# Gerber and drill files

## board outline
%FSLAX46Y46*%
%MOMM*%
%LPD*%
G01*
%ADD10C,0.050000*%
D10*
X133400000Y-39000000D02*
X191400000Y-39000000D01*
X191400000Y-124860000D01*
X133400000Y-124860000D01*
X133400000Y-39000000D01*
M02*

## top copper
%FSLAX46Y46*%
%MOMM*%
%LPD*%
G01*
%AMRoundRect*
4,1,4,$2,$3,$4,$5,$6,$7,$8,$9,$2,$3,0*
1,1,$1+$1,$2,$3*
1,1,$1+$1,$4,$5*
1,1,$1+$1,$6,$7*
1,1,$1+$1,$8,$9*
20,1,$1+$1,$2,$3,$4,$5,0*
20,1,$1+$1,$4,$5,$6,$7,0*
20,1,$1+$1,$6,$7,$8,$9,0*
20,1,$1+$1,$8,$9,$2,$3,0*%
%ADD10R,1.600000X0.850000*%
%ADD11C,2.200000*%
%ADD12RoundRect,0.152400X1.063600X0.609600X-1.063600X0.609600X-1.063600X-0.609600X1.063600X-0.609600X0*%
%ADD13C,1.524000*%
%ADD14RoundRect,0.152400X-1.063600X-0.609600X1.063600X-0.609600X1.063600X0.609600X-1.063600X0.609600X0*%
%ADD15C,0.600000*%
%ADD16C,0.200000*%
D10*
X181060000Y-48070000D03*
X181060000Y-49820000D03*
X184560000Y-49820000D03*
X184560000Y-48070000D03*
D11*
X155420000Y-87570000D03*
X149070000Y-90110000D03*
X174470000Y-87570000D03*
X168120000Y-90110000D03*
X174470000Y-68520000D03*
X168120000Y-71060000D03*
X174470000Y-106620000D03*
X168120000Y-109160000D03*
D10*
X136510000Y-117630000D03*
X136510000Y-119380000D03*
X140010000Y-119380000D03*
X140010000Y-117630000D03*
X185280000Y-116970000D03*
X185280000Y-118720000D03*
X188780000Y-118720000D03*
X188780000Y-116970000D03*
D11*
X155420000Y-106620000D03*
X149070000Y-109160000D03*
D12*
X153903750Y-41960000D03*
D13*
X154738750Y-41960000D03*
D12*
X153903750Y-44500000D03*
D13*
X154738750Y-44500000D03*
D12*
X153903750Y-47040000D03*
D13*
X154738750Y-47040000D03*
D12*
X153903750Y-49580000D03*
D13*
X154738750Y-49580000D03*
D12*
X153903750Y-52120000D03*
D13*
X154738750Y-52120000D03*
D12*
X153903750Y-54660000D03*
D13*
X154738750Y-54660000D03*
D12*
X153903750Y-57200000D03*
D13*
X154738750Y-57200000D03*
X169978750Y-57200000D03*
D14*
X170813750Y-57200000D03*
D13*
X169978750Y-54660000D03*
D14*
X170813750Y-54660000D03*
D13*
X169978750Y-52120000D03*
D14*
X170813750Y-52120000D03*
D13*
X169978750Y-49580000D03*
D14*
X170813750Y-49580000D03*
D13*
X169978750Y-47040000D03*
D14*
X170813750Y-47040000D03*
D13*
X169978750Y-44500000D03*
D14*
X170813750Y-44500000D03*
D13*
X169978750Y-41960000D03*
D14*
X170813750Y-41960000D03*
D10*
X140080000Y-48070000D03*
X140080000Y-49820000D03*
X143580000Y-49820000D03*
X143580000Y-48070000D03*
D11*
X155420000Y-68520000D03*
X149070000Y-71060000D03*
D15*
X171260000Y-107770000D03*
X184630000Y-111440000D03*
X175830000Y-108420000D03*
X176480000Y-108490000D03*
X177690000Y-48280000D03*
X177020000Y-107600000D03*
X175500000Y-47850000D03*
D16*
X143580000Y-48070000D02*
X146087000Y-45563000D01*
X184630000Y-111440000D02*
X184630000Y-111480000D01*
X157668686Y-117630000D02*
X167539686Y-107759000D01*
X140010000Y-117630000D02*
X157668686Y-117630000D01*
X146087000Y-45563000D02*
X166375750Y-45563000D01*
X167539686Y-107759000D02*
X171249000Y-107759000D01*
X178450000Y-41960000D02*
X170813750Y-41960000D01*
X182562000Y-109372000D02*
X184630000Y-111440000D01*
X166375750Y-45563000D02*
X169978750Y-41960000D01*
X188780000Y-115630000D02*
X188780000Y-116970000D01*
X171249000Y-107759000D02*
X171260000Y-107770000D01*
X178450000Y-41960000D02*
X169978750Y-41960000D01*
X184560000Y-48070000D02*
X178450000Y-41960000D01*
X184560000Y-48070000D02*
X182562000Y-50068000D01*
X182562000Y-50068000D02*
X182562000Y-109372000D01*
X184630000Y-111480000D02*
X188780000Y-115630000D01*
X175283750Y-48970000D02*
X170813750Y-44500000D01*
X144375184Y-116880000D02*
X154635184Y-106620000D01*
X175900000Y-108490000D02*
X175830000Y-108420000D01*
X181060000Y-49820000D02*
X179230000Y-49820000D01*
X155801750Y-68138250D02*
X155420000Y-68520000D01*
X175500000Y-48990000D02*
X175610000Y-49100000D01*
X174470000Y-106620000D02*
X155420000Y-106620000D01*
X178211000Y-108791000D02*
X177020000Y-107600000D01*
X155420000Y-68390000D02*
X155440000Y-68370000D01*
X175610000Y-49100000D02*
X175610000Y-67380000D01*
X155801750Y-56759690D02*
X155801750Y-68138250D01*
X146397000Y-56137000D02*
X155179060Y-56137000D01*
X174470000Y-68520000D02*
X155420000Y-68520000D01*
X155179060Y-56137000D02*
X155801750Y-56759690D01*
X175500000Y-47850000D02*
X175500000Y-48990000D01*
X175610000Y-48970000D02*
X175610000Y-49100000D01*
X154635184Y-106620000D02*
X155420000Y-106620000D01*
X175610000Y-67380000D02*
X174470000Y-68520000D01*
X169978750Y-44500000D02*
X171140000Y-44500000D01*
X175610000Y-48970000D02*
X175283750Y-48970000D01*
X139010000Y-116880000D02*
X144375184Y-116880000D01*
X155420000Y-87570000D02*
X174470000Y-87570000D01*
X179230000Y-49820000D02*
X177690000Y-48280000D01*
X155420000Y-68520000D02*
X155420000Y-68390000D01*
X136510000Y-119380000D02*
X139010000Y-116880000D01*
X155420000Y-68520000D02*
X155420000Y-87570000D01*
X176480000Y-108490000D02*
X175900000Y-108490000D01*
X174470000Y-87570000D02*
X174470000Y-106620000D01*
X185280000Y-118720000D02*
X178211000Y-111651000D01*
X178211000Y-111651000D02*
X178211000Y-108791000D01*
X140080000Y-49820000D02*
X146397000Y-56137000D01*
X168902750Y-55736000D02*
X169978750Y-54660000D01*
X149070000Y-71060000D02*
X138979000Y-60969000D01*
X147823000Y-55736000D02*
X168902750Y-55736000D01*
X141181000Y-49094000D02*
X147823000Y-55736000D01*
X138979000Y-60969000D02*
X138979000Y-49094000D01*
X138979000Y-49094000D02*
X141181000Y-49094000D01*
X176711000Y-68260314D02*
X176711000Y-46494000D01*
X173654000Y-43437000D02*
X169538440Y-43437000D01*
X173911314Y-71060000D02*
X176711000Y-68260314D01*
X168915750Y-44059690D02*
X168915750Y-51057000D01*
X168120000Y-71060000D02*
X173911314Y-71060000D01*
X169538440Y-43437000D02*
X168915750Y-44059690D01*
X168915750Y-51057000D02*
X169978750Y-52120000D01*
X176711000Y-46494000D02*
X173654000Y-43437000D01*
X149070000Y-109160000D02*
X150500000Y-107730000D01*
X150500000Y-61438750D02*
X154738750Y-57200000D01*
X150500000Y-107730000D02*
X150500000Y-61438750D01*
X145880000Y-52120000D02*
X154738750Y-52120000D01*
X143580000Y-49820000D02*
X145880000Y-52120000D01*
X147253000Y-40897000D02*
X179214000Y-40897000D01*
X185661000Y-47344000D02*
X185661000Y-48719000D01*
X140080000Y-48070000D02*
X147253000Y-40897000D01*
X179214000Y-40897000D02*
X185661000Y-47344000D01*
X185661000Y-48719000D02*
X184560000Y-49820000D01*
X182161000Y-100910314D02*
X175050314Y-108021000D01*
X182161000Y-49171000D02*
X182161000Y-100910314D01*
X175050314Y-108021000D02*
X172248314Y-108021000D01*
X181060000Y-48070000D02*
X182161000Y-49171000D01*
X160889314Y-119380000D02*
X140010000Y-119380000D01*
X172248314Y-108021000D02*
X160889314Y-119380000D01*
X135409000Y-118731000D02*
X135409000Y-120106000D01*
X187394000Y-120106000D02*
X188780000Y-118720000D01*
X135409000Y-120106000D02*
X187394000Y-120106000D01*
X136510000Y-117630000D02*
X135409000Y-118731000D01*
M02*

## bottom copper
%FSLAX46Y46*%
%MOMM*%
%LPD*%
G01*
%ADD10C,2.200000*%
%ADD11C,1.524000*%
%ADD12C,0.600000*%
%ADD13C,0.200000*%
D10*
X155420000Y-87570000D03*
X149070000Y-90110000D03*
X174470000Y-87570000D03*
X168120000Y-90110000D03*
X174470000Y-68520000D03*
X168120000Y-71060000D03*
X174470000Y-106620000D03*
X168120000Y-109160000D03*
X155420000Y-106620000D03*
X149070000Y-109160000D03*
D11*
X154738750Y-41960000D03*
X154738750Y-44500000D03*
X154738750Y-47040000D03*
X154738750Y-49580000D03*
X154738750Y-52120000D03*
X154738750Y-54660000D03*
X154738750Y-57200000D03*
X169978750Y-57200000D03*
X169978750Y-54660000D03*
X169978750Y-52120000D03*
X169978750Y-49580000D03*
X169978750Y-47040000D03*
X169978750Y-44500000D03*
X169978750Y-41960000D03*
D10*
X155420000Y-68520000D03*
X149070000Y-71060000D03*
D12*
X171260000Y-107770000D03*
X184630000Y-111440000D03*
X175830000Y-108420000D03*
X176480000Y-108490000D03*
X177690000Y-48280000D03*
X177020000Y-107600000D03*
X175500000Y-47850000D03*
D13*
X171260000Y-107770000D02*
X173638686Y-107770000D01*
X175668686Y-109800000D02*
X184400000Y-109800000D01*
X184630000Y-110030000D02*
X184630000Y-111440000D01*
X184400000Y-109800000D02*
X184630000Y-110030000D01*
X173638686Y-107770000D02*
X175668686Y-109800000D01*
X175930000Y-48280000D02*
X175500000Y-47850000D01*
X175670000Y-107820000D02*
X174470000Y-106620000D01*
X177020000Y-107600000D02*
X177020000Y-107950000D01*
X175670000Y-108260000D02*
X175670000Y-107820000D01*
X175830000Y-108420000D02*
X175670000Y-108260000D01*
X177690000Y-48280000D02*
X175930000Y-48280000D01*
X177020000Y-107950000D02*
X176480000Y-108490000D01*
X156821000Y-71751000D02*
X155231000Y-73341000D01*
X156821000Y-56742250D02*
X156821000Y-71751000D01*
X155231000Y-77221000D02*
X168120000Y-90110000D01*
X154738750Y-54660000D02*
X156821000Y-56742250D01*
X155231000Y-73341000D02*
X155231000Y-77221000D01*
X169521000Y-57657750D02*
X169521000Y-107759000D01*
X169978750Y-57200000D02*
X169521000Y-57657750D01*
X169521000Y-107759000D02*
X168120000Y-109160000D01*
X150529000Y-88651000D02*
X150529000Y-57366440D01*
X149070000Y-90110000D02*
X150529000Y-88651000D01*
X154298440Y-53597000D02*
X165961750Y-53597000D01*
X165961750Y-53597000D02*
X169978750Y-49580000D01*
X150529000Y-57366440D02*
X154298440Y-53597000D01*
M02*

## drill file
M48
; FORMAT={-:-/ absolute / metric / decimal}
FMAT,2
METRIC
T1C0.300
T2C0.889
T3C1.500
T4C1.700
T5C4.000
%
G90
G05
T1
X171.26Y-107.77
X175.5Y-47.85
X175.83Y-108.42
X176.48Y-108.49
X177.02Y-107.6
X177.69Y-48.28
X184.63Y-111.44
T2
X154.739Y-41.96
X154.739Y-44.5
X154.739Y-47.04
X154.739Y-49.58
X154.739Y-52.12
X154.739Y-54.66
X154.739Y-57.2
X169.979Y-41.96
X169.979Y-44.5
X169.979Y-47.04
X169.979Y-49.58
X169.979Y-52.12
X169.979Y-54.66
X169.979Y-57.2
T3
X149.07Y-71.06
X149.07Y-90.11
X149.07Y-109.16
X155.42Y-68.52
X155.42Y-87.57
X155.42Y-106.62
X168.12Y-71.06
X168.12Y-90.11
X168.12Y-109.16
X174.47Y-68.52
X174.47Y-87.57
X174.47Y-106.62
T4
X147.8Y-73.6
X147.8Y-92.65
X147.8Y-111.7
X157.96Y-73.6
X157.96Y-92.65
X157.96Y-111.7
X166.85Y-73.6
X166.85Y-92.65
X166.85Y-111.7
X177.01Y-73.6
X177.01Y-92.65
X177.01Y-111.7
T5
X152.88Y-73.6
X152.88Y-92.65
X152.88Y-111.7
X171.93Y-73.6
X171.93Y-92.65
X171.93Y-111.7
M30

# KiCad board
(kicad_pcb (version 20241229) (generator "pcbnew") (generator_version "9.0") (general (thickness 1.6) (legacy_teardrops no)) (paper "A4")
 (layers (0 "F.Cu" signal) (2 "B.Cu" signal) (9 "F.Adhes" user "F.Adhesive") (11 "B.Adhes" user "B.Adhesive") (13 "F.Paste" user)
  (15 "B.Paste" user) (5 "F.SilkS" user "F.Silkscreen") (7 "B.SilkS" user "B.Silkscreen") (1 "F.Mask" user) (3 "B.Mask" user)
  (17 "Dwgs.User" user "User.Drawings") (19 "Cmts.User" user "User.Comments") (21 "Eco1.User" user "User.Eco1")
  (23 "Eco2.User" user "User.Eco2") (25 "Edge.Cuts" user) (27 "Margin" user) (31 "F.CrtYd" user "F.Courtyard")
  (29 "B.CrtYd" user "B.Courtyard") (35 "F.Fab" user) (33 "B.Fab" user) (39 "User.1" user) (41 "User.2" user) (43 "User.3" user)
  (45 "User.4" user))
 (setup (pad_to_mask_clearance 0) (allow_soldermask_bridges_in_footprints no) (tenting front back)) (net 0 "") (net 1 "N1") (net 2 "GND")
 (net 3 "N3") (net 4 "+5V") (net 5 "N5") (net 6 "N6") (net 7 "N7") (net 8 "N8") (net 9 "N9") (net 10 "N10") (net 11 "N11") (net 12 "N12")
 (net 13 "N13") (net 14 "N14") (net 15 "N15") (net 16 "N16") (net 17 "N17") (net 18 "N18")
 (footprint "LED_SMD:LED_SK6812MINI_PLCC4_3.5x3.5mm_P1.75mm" (layer "F.Cu") (at 182.81 48.945)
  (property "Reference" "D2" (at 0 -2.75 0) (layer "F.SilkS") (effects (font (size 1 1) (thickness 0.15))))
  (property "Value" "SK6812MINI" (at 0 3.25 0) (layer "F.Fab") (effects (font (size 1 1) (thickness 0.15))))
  (pad "1" smd rect (at -1.75 -0.875) (size 1.6 0.85) (layers "F.Cu" "F.Mask" "F.Paste") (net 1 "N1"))
  (pad "2" smd rect (at -1.75 0.875) (size 1.6 0.85) (layers "F.Cu" "F.Mask" "F.Paste") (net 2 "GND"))
  (pad "3" smd rect (at 1.75 0.875) (size 1.6 0.85) (layers "F.Cu" "F.Mask" "F.Paste") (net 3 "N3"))
  (pad "4" smd rect (at 1.75 -0.875) (size 1.6 0.85) (layers "F.Cu" "F.Mask" "F.Paste") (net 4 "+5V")))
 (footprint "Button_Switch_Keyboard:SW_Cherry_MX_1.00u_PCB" (layer "F.Cu") (at 155.42 87.57)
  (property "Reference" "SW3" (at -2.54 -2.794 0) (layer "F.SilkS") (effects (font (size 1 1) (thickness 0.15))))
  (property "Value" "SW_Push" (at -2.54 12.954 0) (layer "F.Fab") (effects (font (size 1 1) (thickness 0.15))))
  (pad "" np_thru_hole circle (at -7.62 5.08) (size 1.7 1.7) (drill 1.7) (layers "*.Cu" "*.Mask"))
  (pad "" np_thru_hole circle (at -2.54 5.08) (size 4 4) (drill 4) (layers "*.Cu" "*.Mask"))
  (pad "" np_thru_hole circle (at 2.54 5.08) (size 1.7 1.7) (drill 1.7) (layers "*.Cu" "*.Mask"))
  (pad "1" thru_hole circle (at 0 0) (size 2.2 2.2) (drill 1.5) (layers "*.Cu" "*.Mask") (remove_unused_layers no) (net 2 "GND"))
  (pad "2" thru_hole circle (at -6.35 2.54) (size 2.2 2.2) (drill 1.5) (layers "*.Cu" "*.Mask") (remove_unused_layers no) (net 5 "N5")))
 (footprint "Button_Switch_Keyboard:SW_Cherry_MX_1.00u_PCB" (layer "F.Cu") (at 174.47 87.57)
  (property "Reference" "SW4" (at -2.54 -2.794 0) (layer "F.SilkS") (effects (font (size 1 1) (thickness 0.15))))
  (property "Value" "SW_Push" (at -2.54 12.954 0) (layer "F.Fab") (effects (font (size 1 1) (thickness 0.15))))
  (pad "" np_thru_hole circle (at -7.62 5.08) (size 1.7 1.7) (drill 1.7) (layers "*.Cu" "*.Mask"))
  (pad "" np_thru_hole circle (at -2.54 5.08) (size 4 4) (drill 4) (layers "*.Cu" "*.Mask"))
  (pad "" np_thru_hole circle (at 2.54 5.08) (size 1.7 1.7) (drill 1.7) (layers "*.Cu" "*.Mask"))
  (pad "1" thru_hole circle (at 0 0) (size 2.2 2.2) (drill 1.5) (layers "*.Cu" "*.Mask") (remove_unused_layers no) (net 2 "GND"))
  (pad "2" thru_hole circle (at -6.35 2.54) (size 2.2 2.2) (drill 1.5) (layers "*.Cu" "*.Mask") (remove_unused_layers no) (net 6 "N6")))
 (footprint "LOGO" (layer "F.Cu") (at 187.27 93.68 -90)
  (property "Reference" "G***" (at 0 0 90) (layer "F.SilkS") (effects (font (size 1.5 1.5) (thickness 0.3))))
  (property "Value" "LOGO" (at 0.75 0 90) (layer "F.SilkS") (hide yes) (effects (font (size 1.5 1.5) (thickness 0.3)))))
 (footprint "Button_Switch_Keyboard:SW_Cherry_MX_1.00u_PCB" (layer "F.Cu") (at 174.47 68.52)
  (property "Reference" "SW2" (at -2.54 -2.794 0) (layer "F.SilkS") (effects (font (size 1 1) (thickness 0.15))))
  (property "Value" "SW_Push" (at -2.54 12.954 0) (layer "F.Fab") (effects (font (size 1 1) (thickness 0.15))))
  (pad "" np_thru_hole circle (at -7.62 5.08) (size 1.7 1.7) (drill 1.7) (layers "*.Cu" "*.Mask"))
  (pad "" np_thru_hole circle (at -2.54 5.08) (size 4 4) (drill 4) (layers "*.Cu" "*.Mask"))
  (pad "" np_thru_hole circle (at 2.54 5.08) (size 1.7 1.7) (drill 1.7) (layers "*.Cu" "*.Mask"))
  (pad "1" thru_hole circle (at 0 0) (size 2.2 2.2) (drill 1.5) (layers "*.Cu" "*.Mask") (remove_unused_layers no) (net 2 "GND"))
  (pad "2" thru_hole circle (at -6.35 2.54) (size 2.2 2.2) (drill 1.5) (layers "*.Cu" "*.Mask") (remove_unused_layers no) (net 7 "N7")))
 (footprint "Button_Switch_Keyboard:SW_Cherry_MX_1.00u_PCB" (layer "F.Cu") (at 174.47 106.62)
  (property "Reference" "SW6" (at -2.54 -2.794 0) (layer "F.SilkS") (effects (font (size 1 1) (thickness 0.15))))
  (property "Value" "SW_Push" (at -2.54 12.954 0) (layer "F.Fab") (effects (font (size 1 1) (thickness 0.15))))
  (pad "" np_thru_hole circle (at -7.62 5.08) (size 1.7 1.7) (drill 1.7) (layers "*.Cu" "*.Mask"))
  (pad "" np_thru_hole circle (at -2.54 5.08) (size 4 4) (drill 4) (layers "*.Cu" "*.Mask"))
  (pad "" np_thru_hole circle (at 2.54 5.08) (size 1.7 1.7) (drill 1.7) (layers "*.Cu" "*.Mask"))
  (pad "1" thru_hole circle (at 0 0) (size 2.2 2.2) (drill 1.5) (layers "*.Cu" "*.Mask") (remove_unused_layers no) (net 2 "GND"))
  (pad "2" thru_hole circle (at -6.35 2.54) (size 2.2 2.2) (drill 1.5) (layers "*.Cu" "*.Mask") (remove_unused_layers no) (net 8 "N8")))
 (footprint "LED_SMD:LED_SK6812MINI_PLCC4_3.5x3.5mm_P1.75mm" (layer "F.Cu") (at 138.26 118.505)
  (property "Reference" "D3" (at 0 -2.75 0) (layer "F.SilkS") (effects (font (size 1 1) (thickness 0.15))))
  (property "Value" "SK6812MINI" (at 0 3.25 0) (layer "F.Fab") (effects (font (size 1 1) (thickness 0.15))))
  (pad "1" smd rect (at -1.75 -0.875) (size 1.6 0.85) (layers "F.Cu" "F.Mask" "F.Paste") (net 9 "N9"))
  (pad "2" smd rect (at -1.75 0.875) (size 1.6 0.85) (layers "F.Cu" "F.Mask" "F.Paste") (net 2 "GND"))
  (pad "3" smd rect (at 1.75 0.875) (size 1.6 0.85) (layers "F.Cu" "F.Mask" "F.Paste") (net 1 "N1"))
  (pad "4" smd rect (at 1.75 -0.875) (size 1.6 0.85) (layers "F.Cu" "F.Mask" "F.Paste") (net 4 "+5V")))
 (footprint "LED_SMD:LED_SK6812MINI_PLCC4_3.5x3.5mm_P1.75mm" (layer "F.Cu") (at 187.03 117.845)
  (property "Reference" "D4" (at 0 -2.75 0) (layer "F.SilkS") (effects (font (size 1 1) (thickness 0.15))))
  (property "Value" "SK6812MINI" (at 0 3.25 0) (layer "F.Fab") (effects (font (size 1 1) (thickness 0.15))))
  (pad "1" smd rect (at -1.75 -0.875) (size 1.6 0.85) (layers "F.Cu" "F.Mask" "F.Paste") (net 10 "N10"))
  (pad "2" smd rect (at -1.75 0.875) (size 1.6 0.85) (layers "F.Cu" "F.Mask" "F.Paste") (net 2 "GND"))
  (pad "3" smd rect (at 1.75 0.875) (size 1.6 0.85) (layers "F.Cu" "F.Mask" "F.Paste") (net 9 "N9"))
  (pad "4" smd rect (at 1.75 -0.875) (size 1.6 0.85) (layers "F.Cu" "F.Mask" "F.Paste") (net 4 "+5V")))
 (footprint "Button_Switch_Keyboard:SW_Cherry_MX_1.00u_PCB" (layer "F.Cu") (at 155.42 106.62)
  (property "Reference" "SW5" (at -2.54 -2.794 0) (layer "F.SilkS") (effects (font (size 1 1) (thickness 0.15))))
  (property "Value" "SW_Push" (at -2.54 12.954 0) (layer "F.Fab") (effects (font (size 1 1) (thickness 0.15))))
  (pad "" np_thru_hole circle (at -7.62 5.08) (size 1.7 1.7) (drill 1.7) (layers "*.Cu" "*.Mask"))
  (pad "" np_thru_hole circle (at -2.54 5.08) (size 4 4) (drill 4) (layers "*.Cu" "*.Mask"))
  (pad "" np_thru_hole circle (at 2.54 5.08) (size 1.7 1.7) (drill 1.7) (layers "*.Cu" "*.Mask"))
  (pad "1" thru_hole circle (at 0 0) (size 2.2 2.2) (drill 1.5) (layers "*.Cu" "*.Mask") (remove_unused_layers no) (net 2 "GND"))
  (pad "2" thru_hole circle (at -6.35 2.54) (size 2.2 2.2) (drill 1.5) (layers "*.Cu" "*.Mask") (remove_unused_layers no) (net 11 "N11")))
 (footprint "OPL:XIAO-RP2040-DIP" (layer "F.Cu") (at 162.35875 49.58)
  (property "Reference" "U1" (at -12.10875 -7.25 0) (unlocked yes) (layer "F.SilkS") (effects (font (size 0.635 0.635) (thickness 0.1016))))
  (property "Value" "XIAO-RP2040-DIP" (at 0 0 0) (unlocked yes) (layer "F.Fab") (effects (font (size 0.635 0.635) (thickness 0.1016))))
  (pad "1" smd roundrect (at -8.455 -7.62 180) (size 2.432 1.524) (layers "F.Cu" "F.Mask") (roundrect_rratio 0.1) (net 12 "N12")
   (thermal_bridge_angle 45))
  (pad "1" thru_hole circle (at -7.62 -7.62 180) (size 1.524 1.524) (drill 0.889) (layers "*.Cu" "*.Mask") (remove_unused_layers no)
   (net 12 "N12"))
  (pad "2" smd roundrect (at -8.455 -5.08 180) (size 2.432 1.524) (layers "F.Cu" "F.Mask") (roundrect_rratio 0.1) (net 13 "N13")
   (thermal_bridge_angle 45))
  (pad "2" thru_hole circle (at -7.62 -5.08 180) (size 1.524 1.524) (drill 0.889) (layers "*.Cu" "*.Mask") (remove_unused_layers no)
   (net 13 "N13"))
  (pad "3" smd roundrect (at -8.455 -2.54 180) (size 2.432 1.524) (layers "F.Cu" "F.Mask") (roundrect_rratio 0.1) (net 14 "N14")
   (thermal_bridge_angle 45))
  (pad "3" thru_hole circle (at -7.62 -2.54 180) (size 1.524 1.524) (drill 0.889) (layers "*.Cu" "*.Mask") (remove_unused_layers no)
   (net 14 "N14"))
  (pad "4" smd roundrect (at -8.455 0 180) (size 2.432 1.524) (layers "F.Cu" "F.Mask") (roundrect_rratio 0.1) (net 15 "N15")
   (thermal_bridge_angle 45))
  (pad "4" thru_hole circle (at -7.62 0 180) (size 1.524 1.524) (drill 0.889) (layers "*.Cu" "*.Mask") (remove_unused_layers no)
   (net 15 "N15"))
  (pad "5" smd roundrect (at -8.455 2.54 180) (size 2.432 1.524) (layers "F.Cu" "F.Mask") (roundrect_rratio 0.1) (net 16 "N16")
   (thermal_bridge_angle 45))
  (pad "5" thru_hole circle (at -7.62 2.54 180) (size 1.524 1.524) (drill 0.889) (layers "*.Cu" "*.Mask") (remove_unused_layers no)
   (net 16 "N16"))
  (pad "6" smd roundrect (at -8.455 5.08 180) (size 2.432 1.524) (layers "F.Cu" "F.Mask") (roundrect_rratio 0.1) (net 6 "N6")
   (thermal_bridge_angle 45))
  (pad "6" thru_hole circle (at -7.62 5.08 180) (size 1.524 1.524) (drill 0.889) (layers "*.Cu" "*.Mask") (remove_unused_layers no)
   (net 6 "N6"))
  (pad "7" smd roundrect (at -8.455 7.62 180) (size 2.432 1.524) (layers "F.Cu" "F.Mask") (roundrect_rratio 0.1) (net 11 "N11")
   (thermal_bridge_angle 45))
  (pad "7" thru_hole circle (at -7.62 7.62 180) (size 1.524 1.524) (drill 0.889) (layers "*.Cu" "*.Mask") (remove_unused_layers no)
   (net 11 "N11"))
  (pad "8" thru_hole circle (at 7.62 7.62) (size 1.524 1.524) (drill 0.889) (layers "*.Cu" "*.Mask") (remove_unused_layers no) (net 8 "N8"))
  (pad "8" smd roundrect (at 8.455 7.62) (size 2.432 1.524) (layers "F.Cu" "F.Mask") (roundrect_rratio 0.1) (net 8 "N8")
   (thermal_bridge_angle 45))
  (pad "9" thru_hole circle (at 7.62 5.08) (size 1.524 1.524) (drill 0.889) (layers "*.Cu" "*.Mask") (remove_unused_layers no)
   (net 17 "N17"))
  (pad "9" smd roundrect (at 8.455 5.08) (size 2.432 1.524) (layers "F.Cu" "F.Mask") (roundrect_rratio 0.1) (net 17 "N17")
   (thermal_bridge_angle 45))
  (pad "10" thru_hole circle (at 7.62 2.54) (size 1.524 1.524) (drill 0.889) (layers "*.Cu" "*.Mask") (remove_unused_layers no) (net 7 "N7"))
  (pad "10" smd roundrect (at 8.455 2.54) (size 2.432 1.524) (layers "F.Cu" "F.Mask") (roundrect_rratio 0.1) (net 7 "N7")
   (thermal_bridge_angle 45))
  (pad "11" thru_hole circle (at 7.62 0) (size 1.524 1.524) (drill 0.889) (layers "*.Cu" "*.Mask") (remove_unused_layers no) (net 5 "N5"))
  (pad "11" smd roundrect (at 8.455 0) (size 2.432 1.524) (layers "F.Cu" "F.Mask") (roundrect_rratio 0.1) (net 5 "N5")
   (thermal_bridge_angle 45))
  (pad "12" thru_hole circle (at 7.62 -2.54) (size 1.524 1.524) (drill 0.889) (layers "*.Cu" "*.Mask") (remove_unused_layers no)
   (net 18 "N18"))
  (pad "12" smd roundrect (at 8.455 -2.54) (size 2.432 1.524) (layers "F.Cu" "F.Mask") (roundrect_rratio 0.1) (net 18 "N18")
   (thermal_bridge_angle 45))
  (pad "13" thru_hole circle (at 7.62 -5.08) (size 1.524 1.524) (drill 0.889) (layers "*.Cu" "*.Mask") (remove_unused_layers no)
   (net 2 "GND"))
  (pad "13" smd roundrect (at 8.455 -5.08) (size 2.432 1.524) (layers "F.Cu" "F.Mask") (roundrect_rratio 0.1) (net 2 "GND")
   (thermal_bridge_angle 45))
  (pad "14" thru_hole circle (at 7.62 -7.62) (size 1.524 1.524) (drill 0.889) (layers "*.Cu" "*.Mask") (remove_unused_layers no)
   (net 4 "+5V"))
  (pad "14" smd roundrect (at 8.455 -7.62) (size 2.432 1.524) (layers "F.Cu" "F.Mask") (roundrect_rratio 0.1) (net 4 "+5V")
   (thermal_bridge_angle 45)))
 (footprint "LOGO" (layer "F.Cu") (at 187.310915 74.195059 -90)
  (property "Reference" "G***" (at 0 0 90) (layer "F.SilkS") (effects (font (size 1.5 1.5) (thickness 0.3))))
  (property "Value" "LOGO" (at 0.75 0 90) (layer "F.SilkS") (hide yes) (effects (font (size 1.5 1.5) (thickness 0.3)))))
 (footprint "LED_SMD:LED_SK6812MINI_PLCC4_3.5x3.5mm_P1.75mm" (layer "F.Cu") (at 141.83 48.945)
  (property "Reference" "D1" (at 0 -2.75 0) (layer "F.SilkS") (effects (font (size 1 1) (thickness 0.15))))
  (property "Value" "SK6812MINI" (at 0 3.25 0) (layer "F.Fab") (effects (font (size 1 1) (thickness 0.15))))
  (pad "1" smd rect (at -1.75 -0.875) (size 1.6 0.85) (layers "F.Cu" "F.Mask" "F.Paste") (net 3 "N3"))
  (pad "2" smd rect (at -1.75 0.875) (size 1.6 0.85) (layers "F.Cu" "F.Mask" "F.Paste") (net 2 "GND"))
  (pad "3" smd rect (at 1.75 0.875) (size 1.6 0.85) (layers "F.Cu" "F.Mask" "F.Paste") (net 16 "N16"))
  (pad "4" smd rect (at 1.75 -0.875) (size 1.6 0.85) (layers "F.Cu" "F.Mask" "F.Paste") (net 4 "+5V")))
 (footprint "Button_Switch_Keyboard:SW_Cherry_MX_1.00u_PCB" (layer "F.Cu") (at 155.42 68.52)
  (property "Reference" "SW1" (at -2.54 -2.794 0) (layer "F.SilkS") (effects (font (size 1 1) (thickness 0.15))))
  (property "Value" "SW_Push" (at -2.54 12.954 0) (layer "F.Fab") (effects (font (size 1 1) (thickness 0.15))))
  (pad "" np_thru_hole circle (at -7.62 5.08) (size 1.7 1.7) (drill 1.7) (layers "*.Cu" "*.Mask"))
  (pad "" np_thru_hole circle (at -2.54 5.08) (size 4 4) (drill 4) (layers "*.Cu" "*.Mask"))
  (pad "" np_thru_hole circle (at 2.54 5.08) (size 1.7 1.7) (drill 1.7) (layers "*.Cu" "*.Mask"))
  (pad "1" thru_hole circle (at 0 0) (size 2.2 2.2) (drill 1.5) (layers "*.Cu" "*.Mask") (remove_unused_layers no) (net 2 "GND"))
  (pad "2" thru_hole circle (at -6.35 2.54) (size 2.2 2.2) (drill 1.5) (layers "*.Cu" "*.Mask") (remove_unused_layers no) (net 17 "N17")))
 (gr_rect (start 133.4 39) (end 191.4 124.86) (stroke (width 0.05) (type default)) (fill no) (layer "Edge.Cuts"))
 (segment (start 143.58 48.07) (end 146.087 45.563) (width 0.2) (layer "F.Cu") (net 4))
 (segment (start 184.63 111.44) (end 184.63 111.48) (width 0.2) (layer "F.Cu") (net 4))
 (segment (start 157.668686 117.63) (end 167.539686 107.759) (width 0.2) (layer "F.Cu") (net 4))
 (segment (start 140.01 117.63) (end 157.668686 117.63) (width 0.2) (layer "F.Cu") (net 4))
 (segment (start 146.087 45.563) (end 166.37575 45.563) (width 0.2) (layer "F.Cu") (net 4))
 (segment (start 167.539686 107.759) (end 171.249 107.759) (width 0.2) (layer "F.Cu") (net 4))
 (segment (start 178.45 41.96) (end 170.81375 41.96) (width 0.2) (layer "F.Cu") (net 4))
 (segment (start 182.562 109.372) (end 184.63 111.44) (width 0.2) (layer "F.Cu") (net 4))
 (segment (start 166.37575 45.563) (end 169.97875 41.96) (width 0.2) (layer "F.Cu") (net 4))
 (segment (start 188.78 115.63) (end 188.78 116.97) (width 0.2) (layer "F.Cu") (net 4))
 (segment (start 171.249 107.759) (end 171.26 107.77) (width 0.2) (layer "F.Cu") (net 4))
 (segment (start 178.45 41.96) (end 169.97875 41.96) (width 0.2) (layer "F.Cu") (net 4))
 (segment (start 184.56 48.07) (end 178.45 41.96) (width 0.2) (layer "F.Cu") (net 4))
 (segment (start 184.56 48.07) (end 182.562 50.068) (width 0.2) (layer "F.Cu") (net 4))
 (segment (start 182.562 50.068) (end 182.562 109.372) (width 0.2) (layer "F.Cu") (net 4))
 (segment (start 184.63 111.48) (end 188.78 115.63) (width 0.2) (layer "F.Cu") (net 4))
 (via (at 171.26 107.77) (size 0.6) (drill 0.3) (layers "F.Cu" "B.Cu") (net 4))
 (via (at 184.63 111.44) (size 0.6) (drill 0.3) (layers "F.Cu" "B.Cu") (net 4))
 (segment (start 171.26 107.77) (end 173.638686 107.77) (width 0.2) (layer "B.Cu") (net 4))
 (segment (start 175.668686 109.8) (end 184.4 109.8) (width 0.2) (layer "B.Cu") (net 4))
 (segment (start 184.63 110.03) (end 184.63 111.44) (width 0.2) (layer "B.Cu") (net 4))
 (segment (start 184.4 109.8) (end 184.63 110.03) (width 0.2) (layer "B.Cu") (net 4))
 (segment (start 173.638686 107.77) (end 175.668686 109.8) (width 0.2) (layer "B.Cu") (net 4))
 (segment (start 175.28375 48.97) (end 170.81375 44.5) (width 0.2) (layer "F.Cu") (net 2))
 (segment (start 144.375184 116.88) (end 154.635184 106.62) (width 0.2) (layer "F.Cu") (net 2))
 (segment (start 175.9 108.49) (end 175.83 108.42) (width 0.2) (layer "F.Cu") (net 2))
 (segment (start 181.06 49.82) (end 179.23 49.82) (width 0.2) (layer "F.Cu") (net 2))
 (segment (start 155.80175 68.13825) (end 155.42 68.52) (width 0.2) (layer "F.Cu") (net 2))
 (segment (start 175.5 48.99) (end 175.61 49.1) (width 0.2) (layer "F.Cu") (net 2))
 (segment (start 174.47 106.62) (end 155.42 106.62) (width 0.2) (layer "F.Cu") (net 2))
 (segment (start 178.211 108.791) (end 177.02 107.6) (width 0.2) (layer "F.Cu") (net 2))
 (segment (start 155.42 68.39) (end 155.44 68.37) (width 0.2) (layer "F.Cu") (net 2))
 (segment (start 175.61 49.1) (end 175.61 67.38) (width 0.2) (layer "F.Cu") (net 2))
 (segment (start 155.80175 56.75969) (end 155.80175 68.13825) (width 0.2) (layer "F.Cu") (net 2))
 (segment (start 146.397 56.137) (end 155.17906 56.137) (width 0.2) (layer "F.Cu") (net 2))
 (segment (start 174.47 68.52) (end 155.42 68.52) (width 0.2) (layer "F.Cu") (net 2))
 (segment (start 155.17906 56.137) (end 155.80175 56.75969) (width 0.2) (layer "F.Cu") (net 2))
 (segment (start 175.5 47.85) (end 175.5 48.99) (width 0.2) (layer "F.Cu") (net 2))
 (segment (start 175.61 48.97) (end 175.61 49.1) (width 0.2) (layer "F.Cu") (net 2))
 (segment (start 154.635184 106.62) (end 155.42 106.62) (width 0.2) (layer "F.Cu") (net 2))
 (segment (start 175.61 67.38) (end 174.47 68.52) (width 0.2) (layer "F.Cu") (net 2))
 (segment (start 169.97875 44.5) (end 171.14 44.5) (width 0.2) (layer "F.Cu") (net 2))
 (segment (start 175.61 48.97) (end 175.28375 48.97) (width 0.2) (layer "F.Cu") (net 2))
 (segment (start 139.01 116.88) (end 144.375184 116.88) (width 0.2) (layer "F.Cu") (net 2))
 (segment (start 155.42 87.57) (end 174.47 87.57) (width 0.2) (layer "F.Cu") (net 2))
 (segment (start 179.23 49.82) (end 177.69 48.28) (width 0.2) (layer "F.Cu") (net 2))
 (segment (start 155.42 68.52) (end 155.42 68.39) (width 0.2) (layer "F.Cu") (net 2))
 (segment (start 136.51 119.38) (end 139.01 116.88) (width 0.2) (layer "F.Cu") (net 2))
 (segment (start 155.42 68.52) (end 155.42 87.57) (width 0.2) (layer "F.Cu") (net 2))
 (segment (start 176.48 108.49) (end 175.9 108.49) (width 0.2) (layer "F.Cu") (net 2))
 (segment (start 174.47 87.57) (end 174.47 106.62) (width 0.2) (layer "F.Cu") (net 2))
 (segment (start 185.28 118.72) (end 178.211 111.651) (width 0.2) (layer "F.Cu") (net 2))
 (segment (start 178.211 111.651) (end 178.211 108.791) (width 0.2) (layer "F.Cu") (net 2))
 (segment (start 140.08 49.82) (end 146.397 56.137) (width 0.2) (layer "F.Cu") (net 2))
 (via (at 175.83 108.42) (size 0.6) (drill 0.3) (layers "F.Cu" "B.Cu") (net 2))
 (via (at 176.48 108.49) (size 0.6) (drill 0.3) (layers "F.Cu" "B.Cu") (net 2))
 (via (at 177.69 48.28) (size 0.6) (drill 0.3) (layers "F.Cu" "B.Cu") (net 2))
 (via (at 177.02 107.6) (size 0.6) (drill 0.3) (layers "F.Cu" "B.Cu") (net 2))
 (via (at 175.5 47.85) (size 0.6) (drill 0.3) (layers "F.Cu" "B.Cu") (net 2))
 (segment (start 175.93 48.28) (end 175.5 47.85) (width 0.2) (layer "B.Cu") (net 2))
 (segment (start 175.67 107.82) (end 174.47 106.62) (width 0.2) (layer "B.Cu") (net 2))
 (segment (start 177.02 107.6) (end 177.02 107.95) (width 0.2) (layer "B.Cu") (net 2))
 (segment (start 175.67 108.26) (end 175.67 107.82) (width 0.2) (layer "B.Cu") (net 2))
 (segment (start 175.83 108.42) (end 175.67 108.26) (width 0.2) (layer "B.Cu") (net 2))
 (segment (start 177.69 48.28) (end 175.93 48.28) (width 0.2) (layer "B.Cu") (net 2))
 (segment (start 177.02 107.95) (end 176.48 108.49) (width 0.2) (layer "B.Cu") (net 2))
 (segment (start 168.90275 55.736) (end 169.97875 54.66) (width 0.2) (layer "F.Cu") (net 17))
 (segment (start 149.07 71.06) (end 138.979 60.969) (width 0.2) (layer "F.Cu") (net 17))
 (segment (start 147.823 55.736) (end 168.90275 55.736) (width 0.2) (layer "F.Cu") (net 17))
 (segment (start 141.181 49.094) (end 147.823 55.736) (width 0.2) (layer "F.Cu") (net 17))
 (segment (start 138.979 60.969) (end 138.979 49.094) (width 0.2) (layer "F.Cu") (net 17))
 (segment (start 138.979 49.094) (end 141.181 49.094) (width 0.2) (layer "F.Cu") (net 17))
 (segment (start 176.711 68.260314) (end 176.711 46.494) (width 0.2) (layer "F.Cu") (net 7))
 (segment (start 173.654 43.437) (end 169.53844 43.437) (width 0.2) (layer "F.Cu") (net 7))
 (segment (start 173.911314 71.06) (end 176.711 68.260314) (width 0.2) (layer "F.Cu") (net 7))
 (segment (start 168.91575 44.05969) (end 168.91575 51.057) (width 0.2) (layer "F.Cu") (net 7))
 (segment (start 168.12 71.06) (end 173.911314 71.06) (width 0.2) (layer "F.Cu") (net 7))
 (segment (start 169.53844 43.437) (end 168.91575 44.05969) (width 0.2) (layer "F.Cu") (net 7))
 (segment (start 168.91575 51.057) (end 169.97875 52.12) (width 0.2) (layer "F.Cu") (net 7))
 (segment (start 176.711 46.494) (end 173.654 43.437) (width 0.2) (layer "F.Cu") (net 7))
 (segment (start 156.821 71.751) (end 155.231 73.341) (width 0.2) (layer "B.Cu") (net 6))
 (segment (start 156.821 56.74225) (end 156.821 71.751) (width 0.2) (layer "B.Cu") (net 6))
 (segment (start 155.231 77.221) (end 168.12 90.11) (width 0.2) (layer "B.Cu") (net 6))
 (segment (start 154.73875 54.66) (end 156.821 56.74225) (width 0.2) (layer "B.Cu") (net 6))
 (segment (start 155.231 73.341) (end 155.231 77.221) (width 0.2) (layer "B.Cu") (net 6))
 (segment (start 149.07 109.16) (end 150.5 107.73) (width 0.2) (layer "F.Cu") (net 11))
 (segment (start 150.5 61.43875) (end 154.73875 57.2) (width 0.2) (layer "F.Cu") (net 11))
 (segment (start 150.5 107.73) (end 150.5 61.43875) (width 0.2) (layer "F.Cu") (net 11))
 (segment (start 169.521 57.65775) (end 169.521 107.759) (width 0.2) (layer "B.Cu") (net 8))
 (segment (start 169.97875 57.2) (end 169.521 57.65775) (width 0.2) (layer "B.Cu") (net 8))
 (segment (start 169.521 107.759) (end 168.12 109.16) (width 0.2) (layer "B.Cu") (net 8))
 (segment (start 150.529 88.651) (end 150.529 57.36644) (width 0.2) (layer "B.Cu") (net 5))
 (segment (start 149.07 90.11) (end 150.529 88.651) (width 0.2) (layer "B.Cu") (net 5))
 (segment (start 154.29844 53.597) (end 165.96175 53.597) (width 0.2) (layer "B.Cu") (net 5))
 (segment (start 165.96175 53.597) (end 169.97875 49.58) (width 0.2) (layer "B.Cu") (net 5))
 (segment (start 150.529 57.36644) (end 154.29844 53.597) (width 0.2) (layer "B.Cu") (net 5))
 (segment (start 145.88 52.12) (end 154.73875 52.12) (width 0.2) (layer "F.Cu") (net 16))
 (segment (start 143.58 49.82) (end 145.88 52.12) (width 0.2) (layer "F.Cu") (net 16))
 (segment (start 147.253 40.897) (end 179.214 40.897) (width 0.2) (layer "F.Cu") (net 3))
 (segment (start 185.661 47.344) (end 185.661 48.719) (width 0.2) (layer "F.Cu") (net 3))
 (segment (start 140.08 48.07) (end 147.253 40.897) (width 0.2) (layer "F.Cu") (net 3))
 (segment (start 179.214 40.897) (end 185.661 47.344) (width 0.2) (layer "F.Cu") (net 3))
 (segment (start 185.661 48.719) (end 184.56 49.82) (width 0.2) (layer "F.Cu") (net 3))
 (segment (start 182.161 100.910314) (end 175.050314 108.021) (width 0.2) (layer "F.Cu") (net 1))
 (segment (start 182.161 49.171) (end 182.161 100.910314) (width 0.2) (layer "F.Cu") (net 1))
 (segment (start 175.050314 108.021) (end 172.248314 108.021) (width 0.2) (layer "F.Cu") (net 1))
 (segment (start 181.06 48.07) (end 182.161 49.171) (width 0.2) (layer "F.Cu") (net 1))
 (segment (start 160.889314 119.38) (end 140.01 119.38) (width 0.2) (layer "F.Cu") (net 1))
 (segment (start 172.248314 108.021) (end 160.889314 119.38) (width 0.2) (layer "F.Cu") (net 1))
 (segment (start 135.409 118.731) (end 135.409 120.106) (width 0.2) (layer "F.Cu") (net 9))
 (segment (start 187.394 120.106) (end 188.78 118.72) (width 0.2) (layer "F.Cu") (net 9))
 (segment (start 135.409 120.106) (end 187.394 120.106) (width 0.2) (layer "F.Cu") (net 9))
 (segment (start 136.51 117.63) (end 135.409 118.731) (width 0.2) (layer "F.Cu") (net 9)))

